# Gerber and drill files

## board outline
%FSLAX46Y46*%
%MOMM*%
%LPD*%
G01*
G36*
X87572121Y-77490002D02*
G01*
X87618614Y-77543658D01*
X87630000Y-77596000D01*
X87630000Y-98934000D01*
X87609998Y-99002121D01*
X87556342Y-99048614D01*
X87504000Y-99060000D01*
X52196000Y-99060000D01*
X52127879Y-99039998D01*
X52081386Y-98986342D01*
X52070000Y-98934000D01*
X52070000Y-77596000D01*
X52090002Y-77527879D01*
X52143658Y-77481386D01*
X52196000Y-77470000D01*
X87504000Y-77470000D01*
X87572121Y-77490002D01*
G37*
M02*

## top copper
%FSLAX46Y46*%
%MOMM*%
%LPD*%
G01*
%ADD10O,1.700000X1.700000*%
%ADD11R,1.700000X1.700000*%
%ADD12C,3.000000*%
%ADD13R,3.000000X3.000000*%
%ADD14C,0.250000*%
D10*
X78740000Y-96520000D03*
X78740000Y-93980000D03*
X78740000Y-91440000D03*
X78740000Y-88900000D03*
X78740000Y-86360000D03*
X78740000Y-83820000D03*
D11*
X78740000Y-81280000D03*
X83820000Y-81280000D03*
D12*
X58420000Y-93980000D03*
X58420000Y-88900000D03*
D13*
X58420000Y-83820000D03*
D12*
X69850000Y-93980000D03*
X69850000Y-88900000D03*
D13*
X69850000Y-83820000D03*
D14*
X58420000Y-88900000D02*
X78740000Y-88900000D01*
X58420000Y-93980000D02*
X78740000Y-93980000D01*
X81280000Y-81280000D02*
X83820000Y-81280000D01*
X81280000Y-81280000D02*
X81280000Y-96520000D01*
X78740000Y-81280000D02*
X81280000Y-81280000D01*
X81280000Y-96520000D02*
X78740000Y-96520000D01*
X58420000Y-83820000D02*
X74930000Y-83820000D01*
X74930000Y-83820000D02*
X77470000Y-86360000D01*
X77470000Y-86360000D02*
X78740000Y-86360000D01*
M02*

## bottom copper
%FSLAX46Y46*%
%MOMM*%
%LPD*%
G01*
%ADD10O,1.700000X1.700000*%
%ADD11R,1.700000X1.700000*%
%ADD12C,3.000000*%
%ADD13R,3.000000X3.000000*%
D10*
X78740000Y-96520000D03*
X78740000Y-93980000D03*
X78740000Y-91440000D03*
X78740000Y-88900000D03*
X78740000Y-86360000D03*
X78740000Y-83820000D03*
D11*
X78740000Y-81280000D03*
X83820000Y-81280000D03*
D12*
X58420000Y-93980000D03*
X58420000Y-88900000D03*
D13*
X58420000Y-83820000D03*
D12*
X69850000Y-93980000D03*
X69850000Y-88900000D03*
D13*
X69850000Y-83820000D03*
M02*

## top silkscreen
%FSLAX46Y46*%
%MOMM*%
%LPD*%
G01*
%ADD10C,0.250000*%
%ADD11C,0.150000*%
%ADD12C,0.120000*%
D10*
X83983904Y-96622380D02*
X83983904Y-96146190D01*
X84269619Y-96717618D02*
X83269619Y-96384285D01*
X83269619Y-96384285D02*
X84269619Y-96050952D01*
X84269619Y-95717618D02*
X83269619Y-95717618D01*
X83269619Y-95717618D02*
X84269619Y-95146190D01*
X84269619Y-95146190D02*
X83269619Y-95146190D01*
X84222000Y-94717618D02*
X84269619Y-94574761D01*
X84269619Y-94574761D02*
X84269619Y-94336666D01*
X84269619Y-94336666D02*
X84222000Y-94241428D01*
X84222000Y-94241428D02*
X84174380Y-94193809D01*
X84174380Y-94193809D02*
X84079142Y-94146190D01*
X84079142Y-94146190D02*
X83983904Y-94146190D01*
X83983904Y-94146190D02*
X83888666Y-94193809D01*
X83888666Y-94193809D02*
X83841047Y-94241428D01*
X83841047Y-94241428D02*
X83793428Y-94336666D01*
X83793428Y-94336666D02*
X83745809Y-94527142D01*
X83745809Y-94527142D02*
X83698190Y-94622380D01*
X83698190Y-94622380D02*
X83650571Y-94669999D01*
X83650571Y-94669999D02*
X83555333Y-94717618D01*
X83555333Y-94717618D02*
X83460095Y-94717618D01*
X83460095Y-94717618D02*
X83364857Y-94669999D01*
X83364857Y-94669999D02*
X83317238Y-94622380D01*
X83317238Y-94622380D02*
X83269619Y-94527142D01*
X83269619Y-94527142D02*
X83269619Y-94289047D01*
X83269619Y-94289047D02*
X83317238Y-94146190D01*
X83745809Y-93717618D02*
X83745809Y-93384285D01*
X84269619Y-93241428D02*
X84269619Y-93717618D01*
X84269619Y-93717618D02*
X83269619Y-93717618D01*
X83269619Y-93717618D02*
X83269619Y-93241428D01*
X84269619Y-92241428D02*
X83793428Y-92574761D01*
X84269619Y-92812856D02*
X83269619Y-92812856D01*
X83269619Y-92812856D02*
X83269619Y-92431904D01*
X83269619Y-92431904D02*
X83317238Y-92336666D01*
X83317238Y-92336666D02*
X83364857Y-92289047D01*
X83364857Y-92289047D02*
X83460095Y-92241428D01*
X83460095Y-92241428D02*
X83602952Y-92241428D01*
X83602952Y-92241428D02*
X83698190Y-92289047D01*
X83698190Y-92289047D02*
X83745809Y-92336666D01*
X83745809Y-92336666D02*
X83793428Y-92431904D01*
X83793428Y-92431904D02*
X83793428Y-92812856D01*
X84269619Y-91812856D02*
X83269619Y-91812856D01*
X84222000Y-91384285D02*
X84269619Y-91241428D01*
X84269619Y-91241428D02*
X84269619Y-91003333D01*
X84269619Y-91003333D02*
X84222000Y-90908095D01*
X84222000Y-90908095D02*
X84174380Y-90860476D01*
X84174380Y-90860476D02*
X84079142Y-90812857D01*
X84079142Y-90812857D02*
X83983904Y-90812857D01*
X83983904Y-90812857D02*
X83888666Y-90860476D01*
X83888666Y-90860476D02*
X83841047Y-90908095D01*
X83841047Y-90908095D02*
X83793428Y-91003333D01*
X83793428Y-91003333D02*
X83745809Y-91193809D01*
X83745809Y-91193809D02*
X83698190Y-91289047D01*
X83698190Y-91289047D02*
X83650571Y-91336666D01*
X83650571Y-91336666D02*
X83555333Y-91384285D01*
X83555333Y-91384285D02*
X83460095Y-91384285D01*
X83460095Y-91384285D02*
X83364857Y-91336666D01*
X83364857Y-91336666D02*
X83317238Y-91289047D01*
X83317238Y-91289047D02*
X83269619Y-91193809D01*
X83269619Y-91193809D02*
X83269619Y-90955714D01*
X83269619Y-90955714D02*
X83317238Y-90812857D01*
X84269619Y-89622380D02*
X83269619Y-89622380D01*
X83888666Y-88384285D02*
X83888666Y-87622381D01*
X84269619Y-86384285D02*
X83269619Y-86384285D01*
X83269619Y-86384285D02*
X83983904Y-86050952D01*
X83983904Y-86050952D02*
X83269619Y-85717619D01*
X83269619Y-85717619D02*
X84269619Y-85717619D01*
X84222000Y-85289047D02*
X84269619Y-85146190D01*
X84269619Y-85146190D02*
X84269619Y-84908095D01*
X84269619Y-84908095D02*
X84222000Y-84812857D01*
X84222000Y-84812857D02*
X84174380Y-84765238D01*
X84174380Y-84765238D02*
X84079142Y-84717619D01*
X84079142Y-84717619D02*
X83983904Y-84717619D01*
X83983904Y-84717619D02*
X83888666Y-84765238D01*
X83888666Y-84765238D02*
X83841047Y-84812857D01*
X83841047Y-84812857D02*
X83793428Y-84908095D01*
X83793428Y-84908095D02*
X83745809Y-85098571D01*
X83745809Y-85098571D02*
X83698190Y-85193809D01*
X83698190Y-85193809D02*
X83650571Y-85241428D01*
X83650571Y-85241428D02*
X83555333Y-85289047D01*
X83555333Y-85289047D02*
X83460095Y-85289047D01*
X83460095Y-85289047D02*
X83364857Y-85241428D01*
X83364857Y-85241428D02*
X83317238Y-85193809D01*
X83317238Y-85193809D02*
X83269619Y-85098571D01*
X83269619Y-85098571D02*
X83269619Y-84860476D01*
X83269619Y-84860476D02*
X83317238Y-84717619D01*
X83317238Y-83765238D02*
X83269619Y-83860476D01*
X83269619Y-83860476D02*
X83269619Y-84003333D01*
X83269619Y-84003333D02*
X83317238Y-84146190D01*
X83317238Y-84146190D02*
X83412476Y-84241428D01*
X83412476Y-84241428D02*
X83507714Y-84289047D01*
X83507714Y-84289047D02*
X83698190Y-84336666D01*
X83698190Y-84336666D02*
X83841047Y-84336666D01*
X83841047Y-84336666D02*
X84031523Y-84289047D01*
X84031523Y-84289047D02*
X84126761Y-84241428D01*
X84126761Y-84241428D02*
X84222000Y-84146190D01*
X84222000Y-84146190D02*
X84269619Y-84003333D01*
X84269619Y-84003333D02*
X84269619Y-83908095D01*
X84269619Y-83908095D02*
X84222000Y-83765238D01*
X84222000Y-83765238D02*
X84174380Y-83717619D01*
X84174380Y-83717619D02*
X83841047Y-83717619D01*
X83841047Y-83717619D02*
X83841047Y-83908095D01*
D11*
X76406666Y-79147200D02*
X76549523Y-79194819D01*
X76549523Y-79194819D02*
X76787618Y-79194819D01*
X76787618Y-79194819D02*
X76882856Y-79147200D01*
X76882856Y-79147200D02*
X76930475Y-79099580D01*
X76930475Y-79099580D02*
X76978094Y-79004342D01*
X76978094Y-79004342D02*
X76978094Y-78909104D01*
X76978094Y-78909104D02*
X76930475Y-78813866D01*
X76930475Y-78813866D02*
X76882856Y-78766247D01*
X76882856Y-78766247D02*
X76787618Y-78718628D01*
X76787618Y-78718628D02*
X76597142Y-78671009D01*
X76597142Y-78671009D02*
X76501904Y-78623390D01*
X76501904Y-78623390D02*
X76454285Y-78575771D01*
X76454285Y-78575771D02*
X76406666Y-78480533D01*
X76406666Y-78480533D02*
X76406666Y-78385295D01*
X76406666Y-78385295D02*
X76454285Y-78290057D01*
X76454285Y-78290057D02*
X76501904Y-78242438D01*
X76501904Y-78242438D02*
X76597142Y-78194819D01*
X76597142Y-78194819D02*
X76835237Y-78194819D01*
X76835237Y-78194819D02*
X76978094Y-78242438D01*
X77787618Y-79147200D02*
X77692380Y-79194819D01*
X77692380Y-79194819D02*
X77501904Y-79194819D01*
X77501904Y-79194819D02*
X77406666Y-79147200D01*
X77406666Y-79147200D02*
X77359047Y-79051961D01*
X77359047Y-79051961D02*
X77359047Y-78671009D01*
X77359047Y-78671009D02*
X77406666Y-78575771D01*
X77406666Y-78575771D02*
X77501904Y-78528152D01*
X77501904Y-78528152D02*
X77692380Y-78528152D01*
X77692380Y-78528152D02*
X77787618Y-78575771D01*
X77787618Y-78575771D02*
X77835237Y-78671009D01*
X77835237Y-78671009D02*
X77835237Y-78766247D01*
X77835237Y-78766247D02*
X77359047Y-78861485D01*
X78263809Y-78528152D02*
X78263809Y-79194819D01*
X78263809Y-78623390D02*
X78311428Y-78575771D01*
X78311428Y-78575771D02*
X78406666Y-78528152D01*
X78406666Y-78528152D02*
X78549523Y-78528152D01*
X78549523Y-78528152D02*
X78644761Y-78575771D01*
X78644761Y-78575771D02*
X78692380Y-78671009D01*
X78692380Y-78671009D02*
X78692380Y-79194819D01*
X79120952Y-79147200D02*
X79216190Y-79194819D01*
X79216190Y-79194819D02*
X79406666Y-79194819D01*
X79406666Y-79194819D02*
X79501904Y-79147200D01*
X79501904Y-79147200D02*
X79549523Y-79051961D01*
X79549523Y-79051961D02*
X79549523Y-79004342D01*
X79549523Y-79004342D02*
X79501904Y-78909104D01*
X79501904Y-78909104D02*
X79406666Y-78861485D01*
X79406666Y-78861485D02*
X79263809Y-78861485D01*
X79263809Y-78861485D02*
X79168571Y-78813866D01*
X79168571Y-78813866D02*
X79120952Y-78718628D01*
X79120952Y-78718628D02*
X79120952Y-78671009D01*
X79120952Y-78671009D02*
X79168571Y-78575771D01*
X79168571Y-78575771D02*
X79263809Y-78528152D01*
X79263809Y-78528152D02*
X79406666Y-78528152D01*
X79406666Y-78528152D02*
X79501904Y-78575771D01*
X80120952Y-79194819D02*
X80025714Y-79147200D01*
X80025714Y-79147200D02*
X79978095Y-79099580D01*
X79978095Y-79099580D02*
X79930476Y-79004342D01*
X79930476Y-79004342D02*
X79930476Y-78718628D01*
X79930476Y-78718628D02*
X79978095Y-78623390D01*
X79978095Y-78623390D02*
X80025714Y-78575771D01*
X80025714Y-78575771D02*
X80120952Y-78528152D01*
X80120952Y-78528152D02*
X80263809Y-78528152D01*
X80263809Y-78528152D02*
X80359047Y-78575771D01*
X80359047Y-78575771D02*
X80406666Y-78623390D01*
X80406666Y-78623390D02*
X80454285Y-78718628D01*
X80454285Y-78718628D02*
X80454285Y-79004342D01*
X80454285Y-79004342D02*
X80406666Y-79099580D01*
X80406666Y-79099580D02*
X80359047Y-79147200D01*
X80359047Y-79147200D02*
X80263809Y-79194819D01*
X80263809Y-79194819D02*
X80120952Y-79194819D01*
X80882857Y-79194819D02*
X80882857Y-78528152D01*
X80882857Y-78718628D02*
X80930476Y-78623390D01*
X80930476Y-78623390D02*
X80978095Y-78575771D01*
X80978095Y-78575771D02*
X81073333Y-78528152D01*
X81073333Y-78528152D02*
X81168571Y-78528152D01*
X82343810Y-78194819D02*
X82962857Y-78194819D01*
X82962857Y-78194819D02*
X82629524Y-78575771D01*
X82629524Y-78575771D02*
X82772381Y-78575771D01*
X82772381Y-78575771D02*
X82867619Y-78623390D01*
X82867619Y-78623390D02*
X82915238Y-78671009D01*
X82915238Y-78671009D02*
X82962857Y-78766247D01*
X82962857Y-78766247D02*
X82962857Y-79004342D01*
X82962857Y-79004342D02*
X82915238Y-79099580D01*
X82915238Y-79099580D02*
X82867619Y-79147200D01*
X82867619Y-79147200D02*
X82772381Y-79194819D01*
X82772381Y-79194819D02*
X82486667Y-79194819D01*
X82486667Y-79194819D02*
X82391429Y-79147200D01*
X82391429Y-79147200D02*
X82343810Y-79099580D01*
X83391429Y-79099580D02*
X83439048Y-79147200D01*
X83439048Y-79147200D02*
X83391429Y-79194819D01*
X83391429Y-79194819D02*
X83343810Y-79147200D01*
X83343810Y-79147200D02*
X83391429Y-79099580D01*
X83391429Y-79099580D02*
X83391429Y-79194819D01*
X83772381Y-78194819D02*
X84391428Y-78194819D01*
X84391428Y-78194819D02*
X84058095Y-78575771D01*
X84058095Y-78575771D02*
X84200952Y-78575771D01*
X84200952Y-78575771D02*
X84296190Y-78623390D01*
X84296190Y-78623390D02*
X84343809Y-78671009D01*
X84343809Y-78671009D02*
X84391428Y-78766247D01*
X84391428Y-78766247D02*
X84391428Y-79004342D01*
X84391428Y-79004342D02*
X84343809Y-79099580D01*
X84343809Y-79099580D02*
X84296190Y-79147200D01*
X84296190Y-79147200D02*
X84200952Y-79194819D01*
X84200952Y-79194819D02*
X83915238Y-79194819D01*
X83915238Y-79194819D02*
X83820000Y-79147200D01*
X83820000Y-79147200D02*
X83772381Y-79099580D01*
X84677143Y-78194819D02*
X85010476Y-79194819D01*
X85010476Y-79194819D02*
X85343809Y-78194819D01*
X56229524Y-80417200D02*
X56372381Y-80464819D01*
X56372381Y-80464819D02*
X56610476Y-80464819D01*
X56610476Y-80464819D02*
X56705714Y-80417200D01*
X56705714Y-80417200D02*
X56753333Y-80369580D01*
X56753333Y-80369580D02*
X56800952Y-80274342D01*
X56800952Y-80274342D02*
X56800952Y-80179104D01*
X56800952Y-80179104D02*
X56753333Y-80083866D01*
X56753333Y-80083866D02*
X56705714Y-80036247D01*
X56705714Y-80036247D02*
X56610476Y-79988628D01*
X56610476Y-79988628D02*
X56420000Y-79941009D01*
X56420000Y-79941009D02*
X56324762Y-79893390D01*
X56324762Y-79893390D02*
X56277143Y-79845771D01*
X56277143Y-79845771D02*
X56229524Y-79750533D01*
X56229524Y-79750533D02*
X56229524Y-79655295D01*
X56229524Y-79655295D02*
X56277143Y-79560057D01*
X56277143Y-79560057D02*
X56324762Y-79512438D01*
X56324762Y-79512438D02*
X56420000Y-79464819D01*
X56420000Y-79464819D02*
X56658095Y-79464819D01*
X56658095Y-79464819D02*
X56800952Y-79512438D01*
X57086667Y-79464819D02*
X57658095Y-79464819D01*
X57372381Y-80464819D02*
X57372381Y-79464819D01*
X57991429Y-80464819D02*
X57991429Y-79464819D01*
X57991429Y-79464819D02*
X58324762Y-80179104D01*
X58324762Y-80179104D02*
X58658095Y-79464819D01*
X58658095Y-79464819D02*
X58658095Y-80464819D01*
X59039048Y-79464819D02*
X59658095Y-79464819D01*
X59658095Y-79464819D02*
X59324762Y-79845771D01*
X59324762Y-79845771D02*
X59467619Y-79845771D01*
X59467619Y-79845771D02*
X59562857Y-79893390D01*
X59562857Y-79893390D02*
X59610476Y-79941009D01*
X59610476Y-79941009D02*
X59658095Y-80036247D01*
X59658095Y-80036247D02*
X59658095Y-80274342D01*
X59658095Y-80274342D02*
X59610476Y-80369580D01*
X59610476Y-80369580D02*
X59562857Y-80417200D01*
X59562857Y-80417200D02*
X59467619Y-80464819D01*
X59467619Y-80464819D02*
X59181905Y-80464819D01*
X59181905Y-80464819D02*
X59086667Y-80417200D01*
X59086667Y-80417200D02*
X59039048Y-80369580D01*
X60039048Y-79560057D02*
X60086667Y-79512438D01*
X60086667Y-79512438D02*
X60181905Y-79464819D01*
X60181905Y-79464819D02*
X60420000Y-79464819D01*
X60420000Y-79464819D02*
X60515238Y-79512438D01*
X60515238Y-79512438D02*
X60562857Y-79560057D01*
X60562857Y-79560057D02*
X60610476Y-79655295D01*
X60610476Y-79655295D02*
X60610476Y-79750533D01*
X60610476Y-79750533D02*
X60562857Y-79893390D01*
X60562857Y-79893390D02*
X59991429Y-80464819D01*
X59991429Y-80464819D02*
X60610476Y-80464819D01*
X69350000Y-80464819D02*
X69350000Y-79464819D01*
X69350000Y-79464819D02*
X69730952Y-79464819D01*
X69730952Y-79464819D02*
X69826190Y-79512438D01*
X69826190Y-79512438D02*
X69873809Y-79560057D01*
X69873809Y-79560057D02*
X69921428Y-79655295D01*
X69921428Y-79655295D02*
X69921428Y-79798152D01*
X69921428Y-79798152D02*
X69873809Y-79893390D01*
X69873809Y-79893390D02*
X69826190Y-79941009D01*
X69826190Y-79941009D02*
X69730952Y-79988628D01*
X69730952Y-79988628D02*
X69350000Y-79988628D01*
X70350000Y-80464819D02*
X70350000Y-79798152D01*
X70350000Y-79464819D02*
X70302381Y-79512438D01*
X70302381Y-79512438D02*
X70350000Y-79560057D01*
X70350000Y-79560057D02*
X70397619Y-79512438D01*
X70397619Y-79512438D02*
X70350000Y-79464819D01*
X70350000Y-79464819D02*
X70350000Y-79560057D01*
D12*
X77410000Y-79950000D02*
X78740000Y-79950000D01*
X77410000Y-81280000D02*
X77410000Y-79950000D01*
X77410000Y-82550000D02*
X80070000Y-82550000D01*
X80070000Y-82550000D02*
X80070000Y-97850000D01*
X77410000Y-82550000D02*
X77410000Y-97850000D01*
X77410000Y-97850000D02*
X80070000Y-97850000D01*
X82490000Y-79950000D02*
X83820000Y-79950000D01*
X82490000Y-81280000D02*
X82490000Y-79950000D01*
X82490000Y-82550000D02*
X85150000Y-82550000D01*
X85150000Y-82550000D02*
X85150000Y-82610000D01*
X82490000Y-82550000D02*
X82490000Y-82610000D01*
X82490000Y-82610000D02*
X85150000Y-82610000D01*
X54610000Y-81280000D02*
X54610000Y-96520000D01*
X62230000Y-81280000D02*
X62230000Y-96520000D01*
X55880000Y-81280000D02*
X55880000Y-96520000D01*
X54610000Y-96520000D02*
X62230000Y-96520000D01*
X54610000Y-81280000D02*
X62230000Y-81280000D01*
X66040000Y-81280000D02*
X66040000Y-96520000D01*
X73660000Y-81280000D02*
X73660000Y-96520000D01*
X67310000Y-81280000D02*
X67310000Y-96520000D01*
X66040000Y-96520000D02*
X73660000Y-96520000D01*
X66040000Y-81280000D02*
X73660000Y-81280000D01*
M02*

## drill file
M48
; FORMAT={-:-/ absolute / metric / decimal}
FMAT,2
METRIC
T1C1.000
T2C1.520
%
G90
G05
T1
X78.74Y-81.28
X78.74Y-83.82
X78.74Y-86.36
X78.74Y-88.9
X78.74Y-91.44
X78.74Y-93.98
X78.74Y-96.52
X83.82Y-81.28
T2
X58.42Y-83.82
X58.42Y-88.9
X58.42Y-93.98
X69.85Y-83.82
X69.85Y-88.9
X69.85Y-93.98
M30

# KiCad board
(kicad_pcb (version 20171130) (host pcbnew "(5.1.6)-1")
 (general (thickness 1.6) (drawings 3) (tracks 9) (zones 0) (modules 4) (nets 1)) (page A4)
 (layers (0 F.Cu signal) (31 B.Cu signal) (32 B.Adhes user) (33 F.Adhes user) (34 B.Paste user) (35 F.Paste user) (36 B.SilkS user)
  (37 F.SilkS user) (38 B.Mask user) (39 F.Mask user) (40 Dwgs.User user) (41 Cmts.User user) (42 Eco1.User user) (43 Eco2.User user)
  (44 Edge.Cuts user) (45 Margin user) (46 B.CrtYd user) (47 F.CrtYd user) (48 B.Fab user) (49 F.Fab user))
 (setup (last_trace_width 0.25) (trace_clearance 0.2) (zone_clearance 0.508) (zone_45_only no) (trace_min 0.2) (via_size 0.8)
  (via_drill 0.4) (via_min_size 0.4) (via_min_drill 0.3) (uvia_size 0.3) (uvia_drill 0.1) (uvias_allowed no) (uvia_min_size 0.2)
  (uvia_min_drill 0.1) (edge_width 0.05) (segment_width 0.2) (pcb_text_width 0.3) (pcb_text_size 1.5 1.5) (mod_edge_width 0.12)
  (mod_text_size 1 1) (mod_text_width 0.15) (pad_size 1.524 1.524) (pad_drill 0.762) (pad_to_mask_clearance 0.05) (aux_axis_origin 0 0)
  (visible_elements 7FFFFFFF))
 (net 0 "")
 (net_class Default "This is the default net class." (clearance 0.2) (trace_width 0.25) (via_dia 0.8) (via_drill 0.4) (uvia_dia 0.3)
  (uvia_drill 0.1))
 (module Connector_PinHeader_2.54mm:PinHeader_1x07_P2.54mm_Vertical (layer F.Cu) (at 78.74 81.28)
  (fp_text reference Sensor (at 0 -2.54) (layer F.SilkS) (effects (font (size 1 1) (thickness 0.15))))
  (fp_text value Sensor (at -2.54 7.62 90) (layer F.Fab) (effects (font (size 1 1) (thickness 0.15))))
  (fp_line (start -1.33 -1.33) (end 0 -1.33) (layer F.SilkS) (width 0.12))
  (fp_line (start -1.33 0) (end -1.33 -1.33) (layer F.SilkS) (width 0.12))
  (fp_line (start -1.33 1.27) (end 1.33 1.27) (layer F.SilkS) (width 0.12))
  (fp_line (start 1.33 1.27) (end 1.33 16.57) (layer F.SilkS) (width 0.12))
  (fp_line (start -1.33 1.27) (end -1.33 16.57) (layer F.SilkS) (width 0.12))
  (fp_line (start -1.33 16.57) (end 1.33 16.57) (layer F.SilkS) (width 0.12))
  (pad 7 thru_hole oval (at 0 15.24) (size 1.7 1.7) (drill 1) (layers *.Cu *.Mask))
  (pad 6 thru_hole oval (at 0 12.7) (size 1.7 1.7) (drill 1) (layers *.Cu *.Mask))
  (pad 5 thru_hole oval (at 0 10.16) (size 1.7 1.7) (drill 1) (layers *.Cu *.Mask))
  (pad 4 thru_hole oval (at 0 7.62) (size 1.7 1.7) (drill 1) (layers *.Cu *.Mask))
  (pad 3 thru_hole oval (at 0 5.08) (size 1.7 1.7) (drill 1) (layers *.Cu *.Mask))
  (pad 2 thru_hole oval (at 0 2.54) (size 1.7 1.7) (drill 1) (layers *.Cu *.Mask))
  (pad 1 thru_hole rect (at 0 0) (size 1.7 1.7) (drill 1) (layers *.Cu *.Mask)))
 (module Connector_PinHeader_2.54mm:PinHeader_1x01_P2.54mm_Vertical (layer F.Cu) (at 83.82 81.28)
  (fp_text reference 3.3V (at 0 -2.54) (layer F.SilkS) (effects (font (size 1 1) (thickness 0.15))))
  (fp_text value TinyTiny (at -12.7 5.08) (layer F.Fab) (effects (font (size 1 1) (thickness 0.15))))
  (fp_line (start -1.33 -1.33) (end 0 -1.33) (layer F.SilkS) (width 0.12))
  (fp_line (start -1.33 0) (end -1.33 -1.33) (layer F.SilkS) (width 0.12))
  (fp_line (start -1.33 1.27) (end 1.33 1.27) (layer F.SilkS) (width 0.12))
  (fp_line (start 1.33 1.27) (end 1.33 1.33) (layer F.SilkS) (width 0.12))
  (fp_line (start -1.33 1.27) (end -1.33 1.33) (layer F.SilkS) (width 0.12))
  (fp_line (start -1.33 1.33) (end 1.33 1.33) (layer F.SilkS) (width 0.12))
  (pad 1 thru_hole rect (at 0 0) (size 1.7 1.7) (drill 1) (layers *.Cu *.Mask)))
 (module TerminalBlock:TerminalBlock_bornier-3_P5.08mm (layer F.Cu) (at 58.42 83.82 270)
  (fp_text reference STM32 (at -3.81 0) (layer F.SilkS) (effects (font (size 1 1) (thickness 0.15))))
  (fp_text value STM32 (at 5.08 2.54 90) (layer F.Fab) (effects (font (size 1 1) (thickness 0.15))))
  (fp_line (start -2.54 3.81) (end 12.7 3.81) (layer F.SilkS) (width 0.12))
  (fp_line (start -2.54 -3.81) (end 12.7 -3.81) (layer F.SilkS) (width 0.12))
  (fp_line (start -2.54 2.54) (end 12.7 2.54) (layer F.SilkS) (width 0.12))
  (fp_line (start 12.7 3.81) (end 12.7 -3.81) (layer F.SilkS) (width 0.12))
  (fp_line (start -2.54 3.81) (end -2.54 -3.81) (layer F.SilkS) (width 0.12))
  (pad 3 thru_hole circle (at 10.16 0 270) (size 3 3) (drill 1.52) (layers *.Cu *.Mask))
  (pad 2 thru_hole circle (at 5.08 0 270) (size 3 3) (drill 1.52) (layers *.Cu *.Mask))
  (pad 1 thru_hole rect (at 0 0 270) (size 3 3) (drill 1.52) (layers *.Cu *.Mask)))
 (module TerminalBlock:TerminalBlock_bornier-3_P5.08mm (layer F.Cu) (at 69.85 83.82 270)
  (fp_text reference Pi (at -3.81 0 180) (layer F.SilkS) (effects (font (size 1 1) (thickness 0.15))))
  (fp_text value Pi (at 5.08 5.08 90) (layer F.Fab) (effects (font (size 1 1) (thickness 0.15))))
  (fp_line (start -2.54 3.81) (end 12.7 3.81) (layer F.SilkS) (width 0.12))
  (fp_line (start -2.54 -3.81) (end 12.7 -3.81) (layer F.SilkS) (width 0.12))
  (fp_line (start -2.54 2.54) (end 12.7 2.54) (layer F.SilkS) (width 0.12))
  (fp_line (start 12.7 3.81) (end 12.7 -3.81) (layer F.SilkS) (width 0.12))
  (fp_line (start -2.54 3.81) (end -2.54 -3.81) (layer F.SilkS) (width 0.12))
  (pad 3 thru_hole circle (at 10.16 0 270) (size 3 3) (drill 1.52) (layers *.Cu *.Mask))
  (pad 2 thru_hole circle (at 5.08 0 270) (size 3 3) (drill 1.52) (layers *.Cu *.Mask))
  (pad 1 thru_hole rect (at 0 0 270) (size 3 3) (drill 1.52) (layers *.Cu *.Mask)))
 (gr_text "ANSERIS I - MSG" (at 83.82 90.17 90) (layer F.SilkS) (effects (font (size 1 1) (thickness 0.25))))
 (segment (start 58.42 88.9) (end 78.74 88.9) (width 0.25) (layer F.Cu) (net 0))
 (segment (start 58.42 93.98) (end 78.74 93.98) (width 0.25) (layer F.Cu) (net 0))
 (segment (start 81.28 81.28) (end 83.82 81.28) (width 0.25) (layer F.Cu) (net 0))
 (segment (start 81.28 81.28) (end 81.28 96.52) (width 0.25) (layer F.Cu) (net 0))
 (segment (start 78.74 81.28) (end 81.28 81.28) (width 0.25) (layer F.Cu) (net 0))
 (segment (start 81.28 96.52) (end 78.74 96.52) (width 0.25) (layer F.Cu) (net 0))
 (segment (start 58.42 83.82) (end 74.93 83.82) (width 0.25) (layer F.Cu) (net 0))
 (segment (start 74.93 83.82) (end 77.47 86.36) (width 0.25) (layer F.Cu) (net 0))
 (segment (start 77.47 86.36) (end 78.74 86.36) (width 0.25) (layer F.Cu) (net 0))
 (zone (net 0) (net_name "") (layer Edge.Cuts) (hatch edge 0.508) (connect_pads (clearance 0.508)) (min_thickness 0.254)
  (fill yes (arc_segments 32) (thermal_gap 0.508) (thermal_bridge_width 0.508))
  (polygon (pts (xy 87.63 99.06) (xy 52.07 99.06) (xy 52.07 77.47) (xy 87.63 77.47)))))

